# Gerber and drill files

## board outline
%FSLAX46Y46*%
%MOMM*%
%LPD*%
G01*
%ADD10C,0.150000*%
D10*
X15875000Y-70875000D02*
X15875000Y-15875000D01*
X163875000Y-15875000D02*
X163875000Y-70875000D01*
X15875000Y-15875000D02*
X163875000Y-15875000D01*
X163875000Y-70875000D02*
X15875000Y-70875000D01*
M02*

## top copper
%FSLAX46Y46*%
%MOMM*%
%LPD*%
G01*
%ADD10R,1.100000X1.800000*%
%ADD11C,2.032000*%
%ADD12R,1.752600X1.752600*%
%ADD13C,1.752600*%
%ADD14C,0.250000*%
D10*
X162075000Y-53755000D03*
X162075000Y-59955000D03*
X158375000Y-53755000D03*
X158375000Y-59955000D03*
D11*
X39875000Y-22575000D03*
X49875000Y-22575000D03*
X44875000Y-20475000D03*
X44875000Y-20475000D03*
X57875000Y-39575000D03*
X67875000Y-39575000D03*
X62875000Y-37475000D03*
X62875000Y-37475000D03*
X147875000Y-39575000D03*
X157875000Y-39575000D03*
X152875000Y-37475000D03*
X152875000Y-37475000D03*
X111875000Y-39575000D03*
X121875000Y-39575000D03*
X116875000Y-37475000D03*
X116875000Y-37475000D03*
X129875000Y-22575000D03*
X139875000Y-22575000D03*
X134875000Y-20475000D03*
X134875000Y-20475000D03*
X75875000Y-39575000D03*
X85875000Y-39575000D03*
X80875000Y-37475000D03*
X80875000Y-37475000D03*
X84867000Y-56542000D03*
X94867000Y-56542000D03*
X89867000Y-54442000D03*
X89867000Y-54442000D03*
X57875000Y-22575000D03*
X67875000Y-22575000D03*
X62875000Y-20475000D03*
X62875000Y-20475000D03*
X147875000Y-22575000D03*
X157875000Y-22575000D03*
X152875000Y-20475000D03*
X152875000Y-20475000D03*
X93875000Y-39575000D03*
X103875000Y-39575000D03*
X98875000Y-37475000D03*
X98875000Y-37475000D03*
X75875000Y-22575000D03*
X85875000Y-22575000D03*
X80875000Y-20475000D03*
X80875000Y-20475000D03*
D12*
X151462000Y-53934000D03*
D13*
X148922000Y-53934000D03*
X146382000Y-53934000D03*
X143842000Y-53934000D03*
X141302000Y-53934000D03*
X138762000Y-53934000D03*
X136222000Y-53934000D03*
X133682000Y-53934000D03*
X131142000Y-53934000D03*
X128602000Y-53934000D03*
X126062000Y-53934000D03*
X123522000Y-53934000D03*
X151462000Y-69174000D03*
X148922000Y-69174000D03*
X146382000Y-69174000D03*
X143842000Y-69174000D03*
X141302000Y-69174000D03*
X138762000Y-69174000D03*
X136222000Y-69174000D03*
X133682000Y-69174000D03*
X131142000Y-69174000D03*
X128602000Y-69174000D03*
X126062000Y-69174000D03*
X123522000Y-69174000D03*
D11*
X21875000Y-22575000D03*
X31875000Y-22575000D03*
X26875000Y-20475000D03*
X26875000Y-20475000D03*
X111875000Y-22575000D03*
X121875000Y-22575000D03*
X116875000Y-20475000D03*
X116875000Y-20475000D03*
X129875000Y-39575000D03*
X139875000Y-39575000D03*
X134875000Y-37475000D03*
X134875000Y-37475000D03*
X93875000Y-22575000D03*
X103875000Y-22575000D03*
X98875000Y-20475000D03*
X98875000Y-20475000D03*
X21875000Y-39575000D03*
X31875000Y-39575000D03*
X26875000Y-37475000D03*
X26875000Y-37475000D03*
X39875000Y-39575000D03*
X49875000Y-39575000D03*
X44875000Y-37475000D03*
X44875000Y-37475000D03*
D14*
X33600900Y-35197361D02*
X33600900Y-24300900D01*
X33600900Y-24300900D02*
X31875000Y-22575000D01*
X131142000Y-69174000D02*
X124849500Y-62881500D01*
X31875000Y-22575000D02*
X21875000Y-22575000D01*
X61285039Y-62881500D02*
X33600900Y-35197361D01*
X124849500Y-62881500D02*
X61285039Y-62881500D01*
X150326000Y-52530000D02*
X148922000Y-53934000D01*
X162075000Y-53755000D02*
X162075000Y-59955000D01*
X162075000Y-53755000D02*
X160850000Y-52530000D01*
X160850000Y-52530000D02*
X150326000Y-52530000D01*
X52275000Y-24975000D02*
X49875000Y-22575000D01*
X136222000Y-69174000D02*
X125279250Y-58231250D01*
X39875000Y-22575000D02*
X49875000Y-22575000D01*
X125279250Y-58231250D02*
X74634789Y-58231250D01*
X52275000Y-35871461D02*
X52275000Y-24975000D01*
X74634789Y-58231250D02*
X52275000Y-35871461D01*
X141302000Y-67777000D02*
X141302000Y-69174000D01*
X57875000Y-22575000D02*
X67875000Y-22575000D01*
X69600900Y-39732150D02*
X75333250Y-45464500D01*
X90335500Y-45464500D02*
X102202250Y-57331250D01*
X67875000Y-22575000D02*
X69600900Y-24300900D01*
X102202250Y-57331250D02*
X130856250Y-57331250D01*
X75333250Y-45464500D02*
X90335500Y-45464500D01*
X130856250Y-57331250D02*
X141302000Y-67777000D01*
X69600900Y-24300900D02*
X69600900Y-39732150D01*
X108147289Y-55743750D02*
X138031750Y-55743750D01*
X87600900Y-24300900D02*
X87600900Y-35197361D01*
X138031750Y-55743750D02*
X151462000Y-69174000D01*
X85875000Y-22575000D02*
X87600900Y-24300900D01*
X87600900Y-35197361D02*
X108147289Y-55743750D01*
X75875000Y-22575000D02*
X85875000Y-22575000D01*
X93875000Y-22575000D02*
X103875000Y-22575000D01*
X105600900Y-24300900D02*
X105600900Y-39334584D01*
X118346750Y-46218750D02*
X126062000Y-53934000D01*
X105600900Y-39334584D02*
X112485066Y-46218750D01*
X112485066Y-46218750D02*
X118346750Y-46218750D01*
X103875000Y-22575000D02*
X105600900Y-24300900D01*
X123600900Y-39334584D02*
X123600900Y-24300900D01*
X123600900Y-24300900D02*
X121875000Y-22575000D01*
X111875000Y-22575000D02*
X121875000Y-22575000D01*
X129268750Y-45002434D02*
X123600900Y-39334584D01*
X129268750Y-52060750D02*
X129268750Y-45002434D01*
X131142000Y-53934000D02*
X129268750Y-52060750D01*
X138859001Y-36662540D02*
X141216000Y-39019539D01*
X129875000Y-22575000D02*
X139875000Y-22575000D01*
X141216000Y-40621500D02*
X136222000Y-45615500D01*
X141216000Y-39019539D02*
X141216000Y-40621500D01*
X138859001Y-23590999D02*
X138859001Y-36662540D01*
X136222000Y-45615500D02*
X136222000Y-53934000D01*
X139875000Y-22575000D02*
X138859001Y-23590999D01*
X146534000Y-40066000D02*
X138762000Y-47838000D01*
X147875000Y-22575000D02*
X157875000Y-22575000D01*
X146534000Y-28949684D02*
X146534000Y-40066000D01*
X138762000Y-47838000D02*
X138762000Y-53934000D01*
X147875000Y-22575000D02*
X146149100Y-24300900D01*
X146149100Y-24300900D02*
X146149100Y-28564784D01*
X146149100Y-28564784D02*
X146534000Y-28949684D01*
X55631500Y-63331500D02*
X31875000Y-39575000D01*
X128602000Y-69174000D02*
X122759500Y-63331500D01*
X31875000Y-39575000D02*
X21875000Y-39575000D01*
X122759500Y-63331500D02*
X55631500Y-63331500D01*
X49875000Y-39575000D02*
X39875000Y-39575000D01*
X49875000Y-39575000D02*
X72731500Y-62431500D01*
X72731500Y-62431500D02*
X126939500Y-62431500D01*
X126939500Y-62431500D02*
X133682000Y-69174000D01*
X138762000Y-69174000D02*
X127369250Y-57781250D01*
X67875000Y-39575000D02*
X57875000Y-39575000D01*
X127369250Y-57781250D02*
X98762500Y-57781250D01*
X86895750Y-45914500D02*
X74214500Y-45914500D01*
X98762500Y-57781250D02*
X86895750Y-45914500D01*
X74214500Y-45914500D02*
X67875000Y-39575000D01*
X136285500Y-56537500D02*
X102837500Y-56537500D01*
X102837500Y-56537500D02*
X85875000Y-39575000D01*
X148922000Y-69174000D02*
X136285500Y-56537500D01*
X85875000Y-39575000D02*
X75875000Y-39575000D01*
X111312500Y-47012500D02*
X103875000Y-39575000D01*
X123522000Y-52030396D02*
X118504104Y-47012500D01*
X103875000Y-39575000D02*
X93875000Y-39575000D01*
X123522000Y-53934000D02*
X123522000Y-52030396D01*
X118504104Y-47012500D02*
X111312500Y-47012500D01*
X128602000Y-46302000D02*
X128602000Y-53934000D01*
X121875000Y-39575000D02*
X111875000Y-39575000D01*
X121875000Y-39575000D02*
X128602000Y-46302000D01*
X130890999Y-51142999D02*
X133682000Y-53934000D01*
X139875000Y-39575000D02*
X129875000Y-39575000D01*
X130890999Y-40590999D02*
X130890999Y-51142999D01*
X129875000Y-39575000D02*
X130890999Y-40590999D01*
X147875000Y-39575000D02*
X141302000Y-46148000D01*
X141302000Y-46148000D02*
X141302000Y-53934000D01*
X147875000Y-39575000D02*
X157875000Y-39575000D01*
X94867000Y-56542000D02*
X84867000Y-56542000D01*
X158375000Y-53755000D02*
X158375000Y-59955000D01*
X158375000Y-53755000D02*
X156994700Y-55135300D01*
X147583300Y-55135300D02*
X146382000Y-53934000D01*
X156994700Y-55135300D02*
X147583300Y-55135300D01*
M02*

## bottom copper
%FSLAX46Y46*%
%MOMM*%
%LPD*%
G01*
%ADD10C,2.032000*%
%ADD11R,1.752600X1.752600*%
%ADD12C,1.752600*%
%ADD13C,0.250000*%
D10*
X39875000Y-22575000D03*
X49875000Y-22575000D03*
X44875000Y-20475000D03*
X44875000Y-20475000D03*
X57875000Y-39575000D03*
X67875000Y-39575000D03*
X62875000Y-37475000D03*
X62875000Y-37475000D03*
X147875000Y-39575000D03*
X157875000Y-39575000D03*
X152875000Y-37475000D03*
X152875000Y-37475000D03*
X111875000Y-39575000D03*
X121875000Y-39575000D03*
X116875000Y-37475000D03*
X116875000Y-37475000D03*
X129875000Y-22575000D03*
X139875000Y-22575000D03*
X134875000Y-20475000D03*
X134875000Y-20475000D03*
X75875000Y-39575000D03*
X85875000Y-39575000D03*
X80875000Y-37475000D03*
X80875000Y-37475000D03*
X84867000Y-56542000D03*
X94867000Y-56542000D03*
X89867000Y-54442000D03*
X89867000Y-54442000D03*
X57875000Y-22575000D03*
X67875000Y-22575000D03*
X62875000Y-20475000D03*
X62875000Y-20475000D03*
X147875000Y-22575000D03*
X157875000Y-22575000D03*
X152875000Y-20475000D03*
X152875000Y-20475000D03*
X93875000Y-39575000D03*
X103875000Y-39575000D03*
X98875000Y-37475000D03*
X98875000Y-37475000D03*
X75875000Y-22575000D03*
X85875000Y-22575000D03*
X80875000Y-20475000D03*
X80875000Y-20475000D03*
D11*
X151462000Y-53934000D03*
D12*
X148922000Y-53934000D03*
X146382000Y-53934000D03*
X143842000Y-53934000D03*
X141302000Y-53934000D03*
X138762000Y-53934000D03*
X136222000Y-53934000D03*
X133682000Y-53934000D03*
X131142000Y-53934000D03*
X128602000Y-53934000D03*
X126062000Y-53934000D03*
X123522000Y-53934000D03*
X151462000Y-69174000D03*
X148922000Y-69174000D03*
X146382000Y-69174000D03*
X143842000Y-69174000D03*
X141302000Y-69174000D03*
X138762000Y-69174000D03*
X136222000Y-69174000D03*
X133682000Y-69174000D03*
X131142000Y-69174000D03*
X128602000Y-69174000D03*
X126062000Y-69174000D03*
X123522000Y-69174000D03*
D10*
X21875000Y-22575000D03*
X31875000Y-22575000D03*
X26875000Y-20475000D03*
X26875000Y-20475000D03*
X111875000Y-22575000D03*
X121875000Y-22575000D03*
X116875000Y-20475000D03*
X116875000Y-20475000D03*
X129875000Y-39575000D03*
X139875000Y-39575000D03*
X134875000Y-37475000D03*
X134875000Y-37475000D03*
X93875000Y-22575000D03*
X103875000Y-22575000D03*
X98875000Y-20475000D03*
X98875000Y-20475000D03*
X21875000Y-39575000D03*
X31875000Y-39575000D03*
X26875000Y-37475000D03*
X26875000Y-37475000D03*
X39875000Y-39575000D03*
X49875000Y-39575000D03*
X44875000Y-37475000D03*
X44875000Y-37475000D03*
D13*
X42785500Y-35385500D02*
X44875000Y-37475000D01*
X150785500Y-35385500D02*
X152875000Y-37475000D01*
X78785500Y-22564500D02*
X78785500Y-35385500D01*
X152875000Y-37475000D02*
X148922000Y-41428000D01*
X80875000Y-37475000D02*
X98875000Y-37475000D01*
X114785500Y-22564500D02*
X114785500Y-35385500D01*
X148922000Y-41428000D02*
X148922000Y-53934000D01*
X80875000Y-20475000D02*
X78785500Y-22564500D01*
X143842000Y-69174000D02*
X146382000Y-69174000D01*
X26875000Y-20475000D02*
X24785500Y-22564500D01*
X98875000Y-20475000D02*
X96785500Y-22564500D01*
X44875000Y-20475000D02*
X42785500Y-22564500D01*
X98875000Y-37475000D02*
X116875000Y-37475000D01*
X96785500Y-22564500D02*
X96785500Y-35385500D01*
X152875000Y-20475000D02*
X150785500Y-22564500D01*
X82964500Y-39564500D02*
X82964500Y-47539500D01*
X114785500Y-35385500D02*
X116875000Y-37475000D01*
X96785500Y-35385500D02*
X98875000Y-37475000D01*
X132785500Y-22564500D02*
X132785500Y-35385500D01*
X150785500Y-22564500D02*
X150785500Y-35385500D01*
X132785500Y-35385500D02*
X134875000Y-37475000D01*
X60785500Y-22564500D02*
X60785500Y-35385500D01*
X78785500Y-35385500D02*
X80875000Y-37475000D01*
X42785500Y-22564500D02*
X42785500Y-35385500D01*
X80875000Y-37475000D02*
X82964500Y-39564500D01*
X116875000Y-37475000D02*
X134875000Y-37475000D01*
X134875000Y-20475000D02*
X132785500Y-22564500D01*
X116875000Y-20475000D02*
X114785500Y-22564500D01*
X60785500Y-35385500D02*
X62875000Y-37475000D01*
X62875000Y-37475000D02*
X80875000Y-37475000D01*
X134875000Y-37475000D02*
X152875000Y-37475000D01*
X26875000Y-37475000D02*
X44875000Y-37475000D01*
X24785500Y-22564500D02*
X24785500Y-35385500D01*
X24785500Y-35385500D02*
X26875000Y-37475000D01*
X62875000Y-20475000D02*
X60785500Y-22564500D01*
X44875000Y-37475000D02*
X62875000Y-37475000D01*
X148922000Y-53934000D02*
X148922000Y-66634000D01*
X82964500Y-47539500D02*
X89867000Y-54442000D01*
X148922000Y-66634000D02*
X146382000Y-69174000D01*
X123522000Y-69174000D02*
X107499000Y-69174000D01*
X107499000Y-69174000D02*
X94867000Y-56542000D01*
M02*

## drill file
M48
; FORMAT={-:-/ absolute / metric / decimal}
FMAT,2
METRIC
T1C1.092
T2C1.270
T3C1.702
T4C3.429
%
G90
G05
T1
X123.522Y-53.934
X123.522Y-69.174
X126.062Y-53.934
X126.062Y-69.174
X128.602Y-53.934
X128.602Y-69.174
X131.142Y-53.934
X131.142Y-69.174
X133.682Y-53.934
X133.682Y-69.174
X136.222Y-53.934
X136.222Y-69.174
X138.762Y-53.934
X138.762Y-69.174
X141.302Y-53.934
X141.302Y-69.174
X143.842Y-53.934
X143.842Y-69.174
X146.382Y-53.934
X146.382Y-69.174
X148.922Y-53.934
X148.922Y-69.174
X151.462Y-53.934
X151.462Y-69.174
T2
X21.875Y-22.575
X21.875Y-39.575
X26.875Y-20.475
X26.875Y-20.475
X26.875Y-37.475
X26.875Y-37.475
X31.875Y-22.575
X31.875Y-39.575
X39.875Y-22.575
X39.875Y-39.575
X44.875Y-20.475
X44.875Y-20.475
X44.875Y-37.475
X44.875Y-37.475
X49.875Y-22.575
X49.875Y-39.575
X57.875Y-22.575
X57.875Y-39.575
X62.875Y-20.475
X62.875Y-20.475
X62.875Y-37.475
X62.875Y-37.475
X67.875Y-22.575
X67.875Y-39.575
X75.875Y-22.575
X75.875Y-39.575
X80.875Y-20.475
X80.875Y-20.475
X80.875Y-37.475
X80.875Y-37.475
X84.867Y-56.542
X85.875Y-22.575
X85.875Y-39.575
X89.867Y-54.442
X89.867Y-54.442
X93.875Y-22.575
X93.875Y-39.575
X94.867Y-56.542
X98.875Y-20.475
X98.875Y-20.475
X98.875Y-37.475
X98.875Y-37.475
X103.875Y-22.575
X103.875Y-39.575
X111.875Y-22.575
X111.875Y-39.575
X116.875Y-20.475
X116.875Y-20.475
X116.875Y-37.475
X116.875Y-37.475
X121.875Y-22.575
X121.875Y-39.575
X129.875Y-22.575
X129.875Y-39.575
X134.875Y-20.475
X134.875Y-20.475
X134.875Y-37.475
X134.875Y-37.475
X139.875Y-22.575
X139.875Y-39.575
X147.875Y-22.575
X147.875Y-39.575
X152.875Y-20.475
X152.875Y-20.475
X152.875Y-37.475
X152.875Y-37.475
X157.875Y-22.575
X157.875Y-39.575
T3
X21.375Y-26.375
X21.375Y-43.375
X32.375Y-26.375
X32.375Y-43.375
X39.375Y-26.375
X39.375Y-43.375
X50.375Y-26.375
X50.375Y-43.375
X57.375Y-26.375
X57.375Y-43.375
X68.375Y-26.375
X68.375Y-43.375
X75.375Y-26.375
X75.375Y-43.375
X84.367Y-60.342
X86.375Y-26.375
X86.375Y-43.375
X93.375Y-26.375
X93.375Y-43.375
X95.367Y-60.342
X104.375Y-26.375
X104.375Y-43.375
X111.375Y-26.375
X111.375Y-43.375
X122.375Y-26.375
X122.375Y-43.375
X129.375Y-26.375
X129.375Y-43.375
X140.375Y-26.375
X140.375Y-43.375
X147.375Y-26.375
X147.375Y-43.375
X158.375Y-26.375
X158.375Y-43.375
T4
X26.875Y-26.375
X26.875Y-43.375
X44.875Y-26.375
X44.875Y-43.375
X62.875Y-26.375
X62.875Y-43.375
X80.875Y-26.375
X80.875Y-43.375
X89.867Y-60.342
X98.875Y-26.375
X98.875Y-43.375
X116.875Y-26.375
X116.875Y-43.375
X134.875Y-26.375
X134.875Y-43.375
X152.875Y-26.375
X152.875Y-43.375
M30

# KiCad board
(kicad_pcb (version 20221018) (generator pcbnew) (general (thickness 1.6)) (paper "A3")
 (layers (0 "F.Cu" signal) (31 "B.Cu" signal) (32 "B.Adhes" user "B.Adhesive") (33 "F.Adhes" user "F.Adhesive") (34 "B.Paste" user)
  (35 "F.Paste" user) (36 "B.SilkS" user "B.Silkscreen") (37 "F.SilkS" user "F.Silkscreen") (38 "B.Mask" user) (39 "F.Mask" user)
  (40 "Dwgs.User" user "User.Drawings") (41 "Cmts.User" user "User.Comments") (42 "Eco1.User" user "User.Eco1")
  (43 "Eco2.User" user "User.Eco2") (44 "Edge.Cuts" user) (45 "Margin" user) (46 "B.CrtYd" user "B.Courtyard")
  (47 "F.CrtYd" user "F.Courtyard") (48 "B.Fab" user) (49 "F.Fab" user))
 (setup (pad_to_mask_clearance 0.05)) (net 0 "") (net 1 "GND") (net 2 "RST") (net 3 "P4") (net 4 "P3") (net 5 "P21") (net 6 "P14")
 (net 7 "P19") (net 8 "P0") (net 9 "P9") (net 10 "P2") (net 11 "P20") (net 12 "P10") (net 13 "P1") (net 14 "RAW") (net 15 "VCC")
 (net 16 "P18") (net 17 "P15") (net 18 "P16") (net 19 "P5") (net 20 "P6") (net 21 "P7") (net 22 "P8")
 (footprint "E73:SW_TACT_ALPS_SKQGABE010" (layer "F.Cu") (at 160.225 56.855 -90)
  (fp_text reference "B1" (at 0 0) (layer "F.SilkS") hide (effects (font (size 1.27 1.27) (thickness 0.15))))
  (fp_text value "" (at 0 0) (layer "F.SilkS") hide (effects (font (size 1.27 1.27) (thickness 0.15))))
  (pad "1" smd rect (at -3.1 -1.85 270) (size 1.8 1.1) (layers "F.Cu" "F.Paste" "F.Mask") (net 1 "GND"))
  (pad "1" smd rect (at 3.1 -1.85 270) (size 1.8 1.1) (layers "F.Cu" "F.Paste" "F.Mask") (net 1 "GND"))
  (pad "2" smd rect (at -3.1 1.85 270) (size 1.8 1.1) (layers "F.Cu" "F.Paste" "F.Mask") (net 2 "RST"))
  (pad "2" smd rect (at 3.1 1.85 270) (size 1.8 1.1) (layers "F.Cu" "F.Paste" "F.Mask") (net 2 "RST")))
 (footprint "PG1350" (layer "F.Cu") (at 44.875 26.375)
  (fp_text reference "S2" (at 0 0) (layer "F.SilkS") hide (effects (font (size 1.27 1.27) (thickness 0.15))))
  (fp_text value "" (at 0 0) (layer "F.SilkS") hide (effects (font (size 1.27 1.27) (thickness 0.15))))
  (pad "" np_thru_hole circle (at -5.5 0) (size 1.7018 1.7018) (drill 1.7018) (layers "*.Cu" "*.Mask"))
  (pad "" np_thru_hole circle (at 0 0) (size 3.429 3.429) (drill 3.429) (layers "*.Cu" "*.Mask"))
  (pad "" np_thru_hole circle (at 5.5 0) (size 1.7018 1.7018) (drill 1.7018) (layers "*.Cu" "*.Mask"))
  (pad "1" thru_hole circle (at -5 -3.8) (size 2.032 2.032) (drill 1.27) (layers "*.Cu" "*.Mask") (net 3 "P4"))
  (pad "1" thru_hole circle (at 5 -3.8) (size 2.032 2.032) (drill 1.27) (layers "*.Cu" "*.Mask") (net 3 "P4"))
  (pad "2" thru_hole circle (at 0 -5.9) (size 2.032 2.032) (drill 1.27) (layers "*.Cu" "*.Mask") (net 1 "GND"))
  (pad "2" thru_hole circle (at 0 -5.9) (size 2.032 2.032) (drill 1.27) (layers "*.Cu" "*.Mask") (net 1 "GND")))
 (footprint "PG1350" (layer "F.Cu") (at 62.875 43.375)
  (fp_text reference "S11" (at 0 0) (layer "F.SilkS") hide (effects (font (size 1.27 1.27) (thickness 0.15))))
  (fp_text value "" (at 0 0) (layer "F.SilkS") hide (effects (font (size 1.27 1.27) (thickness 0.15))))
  (pad "" np_thru_hole circle (at -5.5 0) (size 1.7018 1.7018) (drill 1.7018) (layers "*.Cu" "*.Mask"))
  (pad "" np_thru_hole circle (at 0 0) (size 3.429 3.429) (drill 3.429) (layers "*.Cu" "*.Mask"))
  (pad "" np_thru_hole circle (at 5.5 0) (size 1.7018 1.7018) (drill 1.7018) (layers "*.Cu" "*.Mask"))
  (pad "1" thru_hole circle (at -5 -3.8) (size 2.032 2.032) (drill 1.27) (layers "*.Cu" "*.Mask") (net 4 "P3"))
  (pad "1" thru_hole circle (at 5 -3.8) (size 2.032 2.032) (drill 1.27) (layers "*.Cu" "*.Mask") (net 4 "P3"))
  (pad "2" thru_hole circle (at 0 -5.9) (size 2.032 2.032) (drill 1.27) (layers "*.Cu" "*.Mask") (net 1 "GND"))
  (pad "2" thru_hole circle (at 0 -5.9) (size 2.032 2.032) (drill 1.27) (layers "*.Cu" "*.Mask") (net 1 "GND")))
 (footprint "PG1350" (layer "F.Cu") (at 152.875 43.375)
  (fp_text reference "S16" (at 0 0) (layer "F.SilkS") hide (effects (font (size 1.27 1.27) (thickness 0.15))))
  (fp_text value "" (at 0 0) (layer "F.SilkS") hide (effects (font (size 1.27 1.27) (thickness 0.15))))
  (pad "" np_thru_hole circle (at -5.5 0) (size 1.7018 1.7018) (drill 1.7018) (layers "*.Cu" "*.Mask"))
  (pad "" np_thru_hole circle (at 0 0) (size 3.429 3.429) (drill 3.429) (layers "*.Cu" "*.Mask"))
  (pad "" np_thru_hole circle (at 5.5 0) (size 1.7018 1.7018) (drill 1.7018) (layers "*.Cu" "*.Mask"))
  (pad "1" thru_hole circle (at -5 -3.8) (size 2.032 2.032) (drill 1.27) (layers "*.Cu" "*.Mask") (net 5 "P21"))
  (pad "1" thru_hole circle (at 5 -3.8) (size 2.032 2.032) (drill 1.27) (layers "*.Cu" "*.Mask") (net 5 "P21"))
  (pad "2" thru_hole circle (at 0 -5.9) (size 2.032 2.032) (drill 1.27) (layers "*.Cu" "*.Mask") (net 1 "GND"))
  (pad "2" thru_hole circle (at 0 -5.9) (size 2.032 2.032) (drill 1.27) (layers "*.Cu" "*.Mask") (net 1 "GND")))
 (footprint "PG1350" (layer "F.Cu") (at 116.875 43.375)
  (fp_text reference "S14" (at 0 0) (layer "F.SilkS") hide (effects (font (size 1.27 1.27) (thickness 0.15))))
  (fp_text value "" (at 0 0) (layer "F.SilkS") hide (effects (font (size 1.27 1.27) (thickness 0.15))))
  (pad "" np_thru_hole circle (at -5.5 0) (size 1.7018 1.7018) (drill 1.7018) (layers "*.Cu" "*.Mask"))
  (pad "" np_thru_hole circle (at 0 0) (size 3.429 3.429) (drill 3.429) (layers "*.Cu" "*.Mask"))
  (pad "" np_thru_hole circle (at 5.5 0) (size 1.7018 1.7018) (drill 1.7018) (layers "*.Cu" "*.Mask"))
  (pad "1" thru_hole circle (at -5 -3.8) (size 2.032 2.032) (drill 1.27) (layers "*.Cu" "*.Mask") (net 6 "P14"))
  (pad "1" thru_hole circle (at 5 -3.8) (size 2.032 2.032) (drill 1.27) (layers "*.Cu" "*.Mask") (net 6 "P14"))
  (pad "2" thru_hole circle (at 0 -5.9) (size 2.032 2.032) (drill 1.27) (layers "*.Cu" "*.Mask") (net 1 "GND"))
  (pad "2" thru_hole circle (at 0 -5.9) (size 2.032 2.032) (drill 1.27) (layers "*.Cu" "*.Mask") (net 1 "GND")))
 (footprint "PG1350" (layer "F.Cu") (at 134.875 26.375)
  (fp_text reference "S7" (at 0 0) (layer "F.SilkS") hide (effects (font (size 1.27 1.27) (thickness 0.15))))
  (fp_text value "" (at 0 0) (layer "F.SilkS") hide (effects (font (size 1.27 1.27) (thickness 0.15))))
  (pad "" np_thru_hole circle (at -5.5 0) (size 1.7018 1.7018) (drill 1.7018) (layers "*.Cu" "*.Mask"))
  (pad "" np_thru_hole circle (at 0 0) (size 3.429 3.429) (drill 3.429) (layers "*.Cu" "*.Mask"))
  (pad "" np_thru_hole circle (at 5.5 0) (size 1.7018 1.7018) (drill 1.7018) (layers "*.Cu" "*.Mask"))
  (pad "1" thru_hole circle (at -5 -3.8) (size 2.032 2.032) (drill 1.27) (layers "*.Cu" "*.Mask") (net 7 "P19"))
  (pad "1" thru_hole circle (at 5 -3.8) (size 2.032 2.032) (drill 1.27) (layers "*.Cu" "*.Mask") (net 7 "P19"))
  (pad "2" thru_hole circle (at 0 -5.9) (size 2.032 2.032) (drill 1.27) (layers "*.Cu" "*.Mask") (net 1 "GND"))
  (pad "2" thru_hole circle (at 0 -5.9) (size 2.032 2.032) (drill 1.27) (layers "*.Cu" "*.Mask") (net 1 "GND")))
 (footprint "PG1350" (layer "F.Cu") (at 80.875 43.375)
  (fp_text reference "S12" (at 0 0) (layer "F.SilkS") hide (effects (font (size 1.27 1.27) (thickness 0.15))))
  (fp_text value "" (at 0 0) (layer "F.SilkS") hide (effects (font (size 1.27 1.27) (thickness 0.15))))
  (pad "" np_thru_hole circle (at -5.5 0) (size 1.7018 1.7018) (drill 1.7018) (layers "*.Cu" "*.Mask"))
  (pad "" np_thru_hole circle (at 0 0) (size 3.429 3.429) (drill 3.429) (layers "*.Cu" "*.Mask"))
  (pad "" np_thru_hole circle (at 5.5 0) (size 1.7018 1.7018) (drill 1.7018) (layers "*.Cu" "*.Mask"))
  (pad "1" thru_hole circle (at -5 -3.8) (size 2.032 2.032) (drill 1.27) (layers "*.Cu" "*.Mask") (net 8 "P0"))
  (pad "1" thru_hole circle (at 5 -3.8) (size 2.032 2.032) (drill 1.27) (layers "*.Cu" "*.Mask") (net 8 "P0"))
  (pad "2" thru_hole circle (at 0 -5.9) (size 2.032 2.032) (drill 1.27) (layers "*.Cu" "*.Mask") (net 1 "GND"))
  (pad "2" thru_hole circle (at 0 -5.9) (size 2.032 2.032) (drill 1.27) (layers "*.Cu" "*.Mask") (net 1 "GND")))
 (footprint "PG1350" (layer "F.Cu") (at 89.867 60.342)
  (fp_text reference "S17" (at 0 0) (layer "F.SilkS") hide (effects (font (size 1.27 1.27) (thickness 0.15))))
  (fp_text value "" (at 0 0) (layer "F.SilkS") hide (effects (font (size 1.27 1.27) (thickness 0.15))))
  (pad "" np_thru_hole circle (at -5.5 0) (size 1.7018 1.7018) (drill 1.7018) (layers "*.Cu" "*.Mask"))
  (pad "" np_thru_hole circle (at 0 0) (size 3.429 3.429) (drill 3.429) (layers "*.Cu" "*.Mask"))
  (pad "" np_thru_hole circle (at 5.5 0) (size 1.7018 1.7018) (drill 1.7018) (layers "*.Cu" "*.Mask"))
  (pad "1" thru_hole circle (at -5 -3.8) (size 2.032 2.032) (drill 1.27) (layers "*.Cu" "*.Mask") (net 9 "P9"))
  (pad "1" thru_hole circle (at 5 -3.8) (size 2.032 2.032) (drill 1.27) (layers "*.Cu" "*.Mask") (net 9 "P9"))
  (pad "2" thru_hole circle (at 0 -5.9) (size 2.032 2.032) (drill 1.27) (layers "*.Cu" "*.Mask") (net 1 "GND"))
  (pad "2" thru_hole circle (at 0 -5.9) (size 2.032 2.032) (drill 1.27) (layers "*.Cu" "*.Mask") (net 1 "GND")))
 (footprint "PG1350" (layer "F.Cu") (at 62.875 26.375)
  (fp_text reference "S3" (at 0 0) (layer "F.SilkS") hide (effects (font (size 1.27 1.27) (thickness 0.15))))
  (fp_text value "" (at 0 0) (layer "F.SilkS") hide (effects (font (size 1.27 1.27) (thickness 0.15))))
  (pad "" np_thru_hole circle (at -5.5 0) (size 1.7018 1.7018) (drill 1.7018) (layers "*.Cu" "*.Mask"))
  (pad "" np_thru_hole circle (at 0 0) (size 3.429 3.429) (drill 3.429) (layers "*.Cu" "*.Mask"))
  (pad "" np_thru_hole circle (at 5.5 0) (size 1.7018 1.7018) (drill 1.7018) (layers "*.Cu" "*.Mask"))
  (pad "1" thru_hole circle (at -5 -3.8) (size 2.032 2.032) (drill 1.27) (layers "*.Cu" "*.Mask") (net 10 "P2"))
  (pad "1" thru_hole circle (at 5 -3.8) (size 2.032 2.032) (drill 1.27) (layers "*.Cu" "*.Mask") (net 10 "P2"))
  (pad "2" thru_hole circle (at 0 -5.9) (size 2.032 2.032) (drill 1.27) (layers "*.Cu" "*.Mask") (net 1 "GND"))
  (pad "2" thru_hole circle (at 0 -5.9) (size 2.032 2.032) (drill 1.27) (layers "*.Cu" "*.Mask") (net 1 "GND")))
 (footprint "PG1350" (layer "F.Cu") (at 152.875 26.375)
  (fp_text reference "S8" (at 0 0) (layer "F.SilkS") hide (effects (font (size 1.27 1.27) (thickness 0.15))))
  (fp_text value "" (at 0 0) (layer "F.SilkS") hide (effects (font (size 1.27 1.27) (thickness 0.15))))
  (pad "" np_thru_hole circle (at -5.5 0) (size 1.7018 1.7018) (drill 1.7018) (layers "*.Cu" "*.Mask"))
  (pad "" np_thru_hole circle (at 0 0) (size 3.429 3.429) (drill 3.429) (layers "*.Cu" "*.Mask"))
  (pad "" np_thru_hole circle (at 5.5 0) (size 1.7018 1.7018) (drill 1.7018) (layers "*.Cu" "*.Mask"))
  (pad "1" thru_hole circle (at -5 -3.8) (size 2.032 2.032) (drill 1.27) (layers "*.Cu" "*.Mask") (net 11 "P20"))
  (pad "1" thru_hole circle (at 5 -3.8) (size 2.032 2.032) (drill 1.27) (layers "*.Cu" "*.Mask") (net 11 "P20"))
  (pad "2" thru_hole circle (at 0 -5.9) (size 2.032 2.032) (drill 1.27) (layers "*.Cu" "*.Mask") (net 1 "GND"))
  (pad "2" thru_hole circle (at 0 -5.9) (size 2.032 2.032) (drill 1.27) (layers "*.Cu" "*.Mask") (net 1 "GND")))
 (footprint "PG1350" (layer "F.Cu") (at 98.875 43.375)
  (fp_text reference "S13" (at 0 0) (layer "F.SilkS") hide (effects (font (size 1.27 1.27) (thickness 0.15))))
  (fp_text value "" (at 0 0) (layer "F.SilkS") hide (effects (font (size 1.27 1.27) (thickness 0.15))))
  (pad "" np_thru_hole circle (at -5.5 0) (size 1.7018 1.7018) (drill 1.7018) (layers "*.Cu" "*.Mask"))
  (pad "" np_thru_hole circle (at 0 0) (size 3.429 3.429) (drill 3.429) (layers "*.Cu" "*.Mask"))
  (pad "" np_thru_hole circle (at 5.5 0) (size 1.7018 1.7018) (drill 1.7018) (layers "*.Cu" "*.Mask"))
  (pad "1" thru_hole circle (at -5 -3.8) (size 2.032 2.032) (drill 1.27) (layers "*.Cu" "*.Mask") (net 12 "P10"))
  (pad "1" thru_hole circle (at 5 -3.8) (size 2.032 2.032) (drill 1.27) (layers "*.Cu" "*.Mask") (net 12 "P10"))
  (pad "2" thru_hole circle (at 0 -5.9) (size 2.032 2.032) (drill 1.27) (layers "*.Cu" "*.Mask") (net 1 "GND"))
  (pad "2" thru_hole circle (at 0 -5.9) (size 2.032 2.032) (drill 1.27) (layers "*.Cu" "*.Mask") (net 1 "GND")))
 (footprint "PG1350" (layer "F.Cu") (at 80.875 26.375)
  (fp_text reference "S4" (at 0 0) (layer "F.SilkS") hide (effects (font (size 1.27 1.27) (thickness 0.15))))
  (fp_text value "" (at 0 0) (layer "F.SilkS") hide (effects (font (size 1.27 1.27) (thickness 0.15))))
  (pad "" np_thru_hole circle (at -5.5 0) (size 1.7018 1.7018) (drill 1.7018) (layers "*.Cu" "*.Mask"))
  (pad "" np_thru_hole circle (at 0 0) (size 3.429 3.429) (drill 3.429) (layers "*.Cu" "*.Mask"))
  (pad "" np_thru_hole circle (at 5.5 0) (size 1.7018 1.7018) (drill 1.7018) (layers "*.Cu" "*.Mask"))
  (pad "1" thru_hole circle (at -5 -3.8) (size 2.032 2.032) (drill 1.27) (layers "*.Cu" "*.Mask") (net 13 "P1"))
  (pad "1" thru_hole circle (at 5 -3.8) (size 2.032 2.032) (drill 1.27) (layers "*.Cu" "*.Mask") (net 13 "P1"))
  (pad "2" thru_hole circle (at 0 -5.9) (size 2.032 2.032) (drill 1.27) (layers "*.Cu" "*.Mask") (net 1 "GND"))
  (pad "2" thru_hole circle (at 0 -5.9) (size 2.032 2.032) (drill 1.27) (layers "*.Cu" "*.Mask") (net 1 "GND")))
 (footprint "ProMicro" (layer "F.Cu") (at 137.492 61.554 180)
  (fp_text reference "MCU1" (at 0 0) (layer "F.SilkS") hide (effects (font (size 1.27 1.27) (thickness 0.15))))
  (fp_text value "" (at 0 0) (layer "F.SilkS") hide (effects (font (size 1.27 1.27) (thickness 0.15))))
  (pad "1" thru_hole rect (at -13.97 7.62 180) (size 1.7526 1.7526) (drill 1.0922) (layers "*.Cu" "*.SilkS" "*.Mask") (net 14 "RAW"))
  (pad "2" thru_hole circle (at -11.43 7.62 180) (size 1.7526 1.7526) (drill 1.0922) (layers "*.Cu" "*.SilkS" "*.Mask") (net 1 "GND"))
  (pad "3" thru_hole circle (at -8.89 7.62 180) (size 1.7526 1.7526) (drill 1.0922) (layers "*.Cu" "*.SilkS" "*.Mask") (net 2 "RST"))
  (pad "4" thru_hole circle (at -6.35 7.62 180) (size 1.7526 1.7526) (drill 1.0922) (layers "*.Cu" "*.SilkS" "*.Mask") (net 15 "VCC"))
  (pad "5" thru_hole circle (at -3.81 7.62 180) (size 1.7526 1.7526) (drill 1.0922) (layers "*.Cu" "*.SilkS" "*.Mask") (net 5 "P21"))
  (pad "6" thru_hole circle (at -1.27 7.62 180) (size 1.7526 1.7526) (drill 1.0922) (layers "*.Cu" "*.SilkS" "*.Mask") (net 11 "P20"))
  (pad "7" thru_hole circle (at 1.27 7.62 180) (size 1.7526 1.7526) (drill 1.0922) (layers "*.Cu" "*.SilkS" "*.Mask") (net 7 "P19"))
  (pad "8" thru_hole circle (at 3.81 7.62 180) (size 1.7526 1.7526) (drill 1.0922) (layers "*.Cu" "*.SilkS" "*.Mask") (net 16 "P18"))
  (pad "9" thru_hole circle (at 6.35 7.62 180) (size 1.7526 1.7526) (drill 1.0922) (layers "*.Cu" "*.SilkS" "*.Mask") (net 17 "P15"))
  (pad "10" thru_hole circle (at 8.89 7.62 180) (size 1.7526 1.7526) (drill 1.0922) (layers "*.Cu" "*.SilkS" "*.Mask") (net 6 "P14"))
  (pad "11" thru_hole circle (at 11.43 7.62 180) (size 1.7526 1.7526) (drill 1.0922) (layers "*.Cu" "*.SilkS" "*.Mask") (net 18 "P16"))
  (pad "12" thru_hole circle (at 13.97 7.62 180) (size 1.7526 1.7526) (drill 1.0922) (layers "*.Cu" "*.SilkS" "*.Mask") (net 12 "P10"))
  (pad "13" thru_hole circle (at -13.97 -7.62 180) (size 1.7526 1.7526) (drill 1.0922) (layers "*.Cu" "*.SilkS" "*.Mask") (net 13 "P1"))
  (pad "14" thru_hole circle (at -11.43 -7.62 180) (size 1.7526 1.7526) (drill 1.0922) (layers "*.Cu" "*.SilkS" "*.Mask") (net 8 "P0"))
  (pad "15" thru_hole circle (at -8.89 -7.62 180) (size 1.7526 1.7526) (drill 1.0922) (layers "*.Cu" "*.SilkS" "*.Mask") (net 1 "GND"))
  (pad "16" thru_hole circle (at -6.35 -7.62 180) (size 1.7526 1.7526) (drill 1.0922) (layers "*.Cu" "*.SilkS" "*.Mask") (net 1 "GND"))
  (pad "17" thru_hole circle (at -3.81 -7.62 180) (size 1.7526 1.7526) (drill 1.0922) (layers "*.Cu" "*.SilkS" "*.Mask") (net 10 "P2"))
  (pad "18" thru_hole circle (at -1.27 -7.62 180) (size 1.7526 1.7526) (drill 1.0922) (layers "*.Cu" "*.SilkS" "*.Mask") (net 4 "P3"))
  (pad "19" thru_hole circle (at 1.27 -7.62 180) (size 1.7526 1.7526) (drill 1.0922) (layers "*.Cu" "*.SilkS" "*.Mask") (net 3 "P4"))
  (pad "20" thru_hole circle (at 3.81 -7.62 180) (size 1.7526 1.7526) (drill 1.0922) (layers "*.Cu" "*.SilkS" "*.Mask") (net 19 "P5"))
  (pad "21" thru_hole circle (at 6.35 -7.62 180) (size 1.7526 1.7526) (drill 1.0922) (layers "*.Cu" "*.SilkS" "*.Mask") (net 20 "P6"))
  (pad "22" thru_hole circle (at 8.89 -7.62 180) (size 1.7526 1.7526) (drill 1.0922) (layers "*.Cu" "*.SilkS" "*.Mask") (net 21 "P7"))
  (pad "23" thru_hole circle (at 11.43 -7.62 180) (size 1.7526 1.7526) (drill 1.0922) (layers "*.Cu" "*.SilkS" "*.Mask") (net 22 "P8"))
  (pad "24" thru_hole circle (at 13.97 -7.62 180) (size 1.7526 1.7526) (drill 1.0922) (layers "*.Cu" "*.SilkS" "*.Mask") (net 9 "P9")))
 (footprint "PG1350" (layer "F.Cu") (at 26.875 26.375)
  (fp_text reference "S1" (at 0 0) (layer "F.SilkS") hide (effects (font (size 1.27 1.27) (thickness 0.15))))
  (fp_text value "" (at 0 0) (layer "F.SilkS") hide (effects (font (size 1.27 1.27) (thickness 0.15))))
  (pad "" np_thru_hole circle (at -5.5 0) (size 1.7018 1.7018) (drill 1.7018) (layers "*.Cu" "*.Mask"))
  (pad "" np_thru_hole circle (at 0 0) (size 3.429 3.429) (drill 3.429) (layers "*.Cu" "*.Mask"))
  (pad "" np_thru_hole circle (at 5.5 0) (size 1.7018 1.7018) (drill 1.7018) (layers "*.Cu" "*.Mask"))
  (pad "1" thru_hole circle (at -5 -3.8) (size 2.032 2.032) (drill 1.27) (layers "*.Cu" "*.Mask") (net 20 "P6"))
  (pad "1" thru_hole circle (at 5 -3.8) (size 2.032 2.032) (drill 1.27) (layers "*.Cu" "*.Mask") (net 20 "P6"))
  (pad "2" thru_hole circle (at 0 -5.9) (size 2.032 2.032) (drill 1.27) (layers "*.Cu" "*.Mask") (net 1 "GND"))
  (pad "2" thru_hole circle (at 0 -5.9) (size 2.032 2.032) (drill 1.27) (layers "*.Cu" "*.Mask") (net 1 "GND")))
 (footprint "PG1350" (layer "F.Cu") (at 116.875 26.375)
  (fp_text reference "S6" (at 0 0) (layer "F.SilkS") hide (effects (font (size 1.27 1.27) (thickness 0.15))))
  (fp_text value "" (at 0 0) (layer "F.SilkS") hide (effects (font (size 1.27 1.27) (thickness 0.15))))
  (pad "" np_thru_hole circle (at -5.5 0) (size 1.7018 1.7018) (drill 1.7018) (layers "*.Cu" "*.Mask"))
  (pad "" np_thru_hole circle (at 0 0) (size 3.429 3.429) (drill 3.429) (layers "*.Cu" "*.Mask"))
  (pad "" np_thru_hole circle (at 5.5 0) (size 1.7018 1.7018) (drill 1.7018) (layers "*.Cu" "*.Mask"))
  (pad "1" thru_hole circle (at -5 -3.8) (size 2.032 2.032) (drill 1.27) (layers "*.Cu" "*.Mask") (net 17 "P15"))
  (pad "1" thru_hole circle (at 5 -3.8) (size 2.032 2.032) (drill 1.27) (layers "*.Cu" "*.Mask") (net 17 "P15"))
  (pad "2" thru_hole circle (at 0 -5.9) (size 2.032 2.032) (drill 1.27) (layers "*.Cu" "*.Mask") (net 1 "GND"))
  (pad "2" thru_hole circle (at 0 -5.9) (size 2.032 2.032) (drill 1.27) (layers "*.Cu" "*.Mask") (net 1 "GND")))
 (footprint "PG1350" (layer "F.Cu") (at 134.875 43.375)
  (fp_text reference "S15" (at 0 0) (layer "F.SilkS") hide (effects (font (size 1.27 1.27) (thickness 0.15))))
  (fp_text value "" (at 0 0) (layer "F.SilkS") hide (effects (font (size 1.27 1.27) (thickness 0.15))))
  (pad "" np_thru_hole circle (at -5.5 0) (size 1.7018 1.7018) (drill 1.7018) (layers "*.Cu" "*.Mask"))
  (pad "" np_thru_hole circle (at 0 0) (size 3.429 3.429) (drill 3.429) (layers "*.Cu" "*.Mask"))
  (pad "" np_thru_hole circle (at 5.5 0) (size 1.7018 1.7018) (drill 1.7018) (layers "*.Cu" "*.Mask"))
  (pad "1" thru_hole circle (at -5 -3.8) (size 2.032 2.032) (drill 1.27) (layers "*.Cu" "*.Mask") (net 16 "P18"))
  (pad "1" thru_hole circle (at 5 -3.8) (size 2.032 2.032) (drill 1.27) (layers "*.Cu" "*.Mask") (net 16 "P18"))
  (pad "2" thru_hole circle (at 0 -5.9) (size 2.032 2.032) (drill 1.27) (layers "*.Cu" "*.Mask") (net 1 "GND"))
  (pad "2" thru_hole circle (at 0 -5.9) (size 2.032 2.032) (drill 1.27) (layers "*.Cu" "*.Mask") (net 1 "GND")))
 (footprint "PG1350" (layer "F.Cu") (at 98.875 26.375)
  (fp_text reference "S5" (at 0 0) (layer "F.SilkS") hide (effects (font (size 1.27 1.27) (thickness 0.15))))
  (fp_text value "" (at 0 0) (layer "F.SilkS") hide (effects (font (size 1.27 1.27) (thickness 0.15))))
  (pad "" np_thru_hole circle (at -5.5 0) (size 1.7018 1.7018) (drill 1.7018) (layers "*.Cu" "*.Mask"))
  (pad "" np_thru_hole circle (at 0 0) (size 3.429 3.429) (drill 3.429) (layers "*.Cu" "*.Mask"))
  (pad "" np_thru_hole circle (at 5.5 0) (size 1.7018 1.7018) (drill 1.7018) (layers "*.Cu" "*.Mask"))
  (pad "1" thru_hole circle (at -5 -3.8) (size 2.032 2.032) (drill 1.27) (layers "*.Cu" "*.Mask") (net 18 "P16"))
  (pad "1" thru_hole circle (at 5 -3.8) (size 2.032 2.032) (drill 1.27) (layers "*.Cu" "*.Mask") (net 18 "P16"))
  (pad "2" thru_hole circle (at 0 -5.9) (size 2.032 2.032) (drill 1.27) (layers "*.Cu" "*.Mask") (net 1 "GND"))
  (pad "2" thru_hole circle (at 0 -5.9) (size 2.032 2.032) (drill 1.27) (layers "*.Cu" "*.Mask") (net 1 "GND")))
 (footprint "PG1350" (layer "F.Cu") (at 26.875 43.375)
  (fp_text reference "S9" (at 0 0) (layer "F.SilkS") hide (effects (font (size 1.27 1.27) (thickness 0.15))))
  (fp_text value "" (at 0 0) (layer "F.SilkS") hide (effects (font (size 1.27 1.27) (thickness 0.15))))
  (pad "" np_thru_hole circle (at -5.5 0) (size 1.7018 1.7018) (drill 1.7018) (layers "*.Cu" "*.Mask"))
  (pad "" np_thru_hole circle (at 0 0) (size 3.429 3.429) (drill 3.429) (layers "*.Cu" "*.Mask"))
  (pad "" np_thru_hole circle (at 5.5 0) (size 1.7018 1.7018) (drill 1.7018) (layers "*.Cu" "*.Mask"))
  (pad "1" thru_hole circle (at -5 -3.8) (size 2.032 2.032) (drill 1.27) (layers "*.Cu" "*.Mask") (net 21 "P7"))
  (pad "1" thru_hole circle (at 5 -3.8) (size 2.032 2.032) (drill 1.27) (layers "*.Cu" "*.Mask") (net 21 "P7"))
  (pad "2" thru_hole circle (at 0 -5.9) (size 2.032 2.032) (drill 1.27) (layers "*.Cu" "*.Mask") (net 1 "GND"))
  (pad "2" thru_hole circle (at 0 -5.9) (size 2.032 2.032) (drill 1.27) (layers "*.Cu" "*.Mask") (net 1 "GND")))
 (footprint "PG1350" (layer "F.Cu") (at 44.875 43.375)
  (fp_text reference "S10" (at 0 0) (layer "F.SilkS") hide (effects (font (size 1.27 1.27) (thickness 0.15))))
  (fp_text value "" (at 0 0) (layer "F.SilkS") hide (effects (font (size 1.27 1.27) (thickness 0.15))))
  (pad "" np_thru_hole circle (at -5.5 0) (size 1.7018 1.7018) (drill 1.7018) (layers "*.Cu" "*.Mask"))
  (pad "" np_thru_hole circle (at 0 0) (size 3.429 3.429) (drill 3.429) (layers "*.Cu" "*.Mask"))
  (pad "" np_thru_hole circle (at 5.5 0) (size 1.7018 1.7018) (drill 1.7018) (layers "*.Cu" "*.Mask"))
  (pad "1" thru_hole circle (at -5 -3.8) (size 2.032 2.032) (drill 1.27) (layers "*.Cu" "*.Mask") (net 19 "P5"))
  (pad "1" thru_hole circle (at 5 -3.8) (size 2.032 2.032) (drill 1.27) (layers "*.Cu" "*.Mask") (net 19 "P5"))
  (pad "2" thru_hole circle (at 0 -5.9) (size 2.032 2.032) (drill 1.27) (layers "*.Cu" "*.Mask") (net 1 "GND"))
  (pad "2" thru_hole circle (at 0 -5.9) (size 2.032 2.032) (drill 1.27) (layers "*.Cu" "*.Mask") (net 1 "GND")))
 (gr_line (start 15.875 70.875) (end 15.875 15.875) (stroke (width 0.15) (type solid)) (layer "Edge.Cuts"))
 (gr_line (start 163.875 15.875) (end 163.875 70.875) (stroke (width 0.15) (type solid)) (layer "Edge.Cuts"))
 (gr_line (start 15.875 15.875) (end 163.875 15.875) (stroke (width 0.15) (type solid)) (layer "Edge.Cuts"))
 (gr_line (start 163.875 70.875) (end 15.875 70.875) (stroke (width 0.15) (type solid)) (layer "Edge.Cuts"))
 (segment (start 33.6009 35.197361) (end 33.6009 24.3009) (width 0.25) (layer "F.Cu") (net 20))
 (segment (start 33.6009 24.3009) (end 31.875 22.575) (width 0.25) (layer "F.Cu") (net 20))
 (segment (start 131.142 69.174) (end 124.8495 62.8815) (width 0.25) (layer "F.Cu") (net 20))
 (segment (start 31.875 22.575) (end 21.875 22.575) (width 0.25) (layer "F.Cu") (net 20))
 (segment (start 61.285039 62.8815) (end 33.6009 35.197361) (width 0.25) (layer "F.Cu") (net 20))
 (segment (start 124.8495 62.8815) (end 61.285039 62.8815) (width 0.25) (layer "F.Cu") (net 20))
 (segment (start 150.326 52.53) (end 148.922 53.934) (width 0.25) (layer "F.Cu") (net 1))
 (segment (start 162.075 53.755) (end 162.075 59.955) (width 0.25) (layer "F.Cu") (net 1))
 (segment (start 162.075 53.755) (end 160.85 52.53) (width 0.25) (layer "F.Cu") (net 1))
 (segment (start 160.85 52.53) (end 150.326 52.53) (width 0.25) (layer "F.Cu") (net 1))
 (segment (start 42.7855 35.3855) (end 44.875 37.475) (width 0.25) (layer "B.Cu") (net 1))
 (segment (start 150.7855 35.3855) (end 152.875 37.475) (width 0.25) (layer "B.Cu") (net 1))
 (segment (start 78.7855 22.5645) (end 78.7855 35.3855) (width 0.25) (layer "B.Cu") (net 1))
 (segment (start 152.875 37.475) (end 148.922 41.428) (width 0.25) (layer "B.Cu") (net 1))
 (segment (start 80.875 37.475) (end 98.875 37.475) (width 0.25) (layer "B.Cu") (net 1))
 (segment (start 114.7855 22.5645) (end 114.7855 35.3855) (width 0.25) (layer "B.Cu") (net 1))
 (segment (start 148.922 41.428) (end 148.922 53.934) (width 0.25) (layer "B.Cu") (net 1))
 (segment (start 80.875 20.475) (end 78.7855 22.5645) (width 0.25) (layer "B.Cu") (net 1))
 (segment (start 143.842 69.174) (end 146.382 69.174) (width 0.25) (layer "B.Cu") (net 1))
 (segment (start 26.875 20.475) (end 24.7855 22.5645) (width 0.25) (layer "B.Cu") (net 1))
 (segment (start 98.875 20.475) (end 96.7855 22.5645) (width 0.25) (layer "B.Cu") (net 1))
 (segment (start 44.875 20.475) (end 42.7855 22.5645) (width 0.25) (layer "B.Cu") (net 1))
 (segment (start 98.875 37.475) (end 116.875 37.475) (width 0.25) (layer "B.Cu") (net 1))
 (segment (start 96.7855 22.5645) (end 96.7855 35.3855) (width 0.25) (layer "B.Cu") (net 1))
 (segment (start 152.875 20.475) (end 150.7855 22.5645) (width 0.25) (layer "B.Cu") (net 1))
 (segment (start 82.9645 39.5645) (end 82.9645 47.5395) (width 0.25) (layer "B.Cu") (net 1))
 (segment (start 114.7855 35.3855) (end 116.875 37.475) (width 0.25) (layer "B.Cu") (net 1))
 (segment (start 96.7855 35.3855) (end 98.875 37.475) (width 0.25) (layer "B.Cu") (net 1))
 (segment (start 132.7855 22.5645) (end 132.7855 35.3855) (width 0.25) (layer "B.Cu") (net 1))
 (segment (start 150.7855 22.5645) (end 150.7855 35.3855) (width 0.25) (layer "B.Cu") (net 1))
 (segment (start 132.7855 35.3855) (end 134.875 37.475) (width 0.25) (layer "B.Cu") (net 1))
 (segment (start 60.7855 22.5645) (end 60.7855 35.3855) (width 0.25) (layer "B.Cu") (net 1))
 (segment (start 78.7855 35.3855) (end 80.875 37.475) (width 0.25) (layer "B.Cu") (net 1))
 (segment (start 42.7855 22.5645) (end 42.7855 35.3855) (width 0.25) (layer "B.Cu") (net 1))
 (segment (start 80.875 37.475) (end 82.9645 39.5645) (width 0.25) (layer "B.Cu") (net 1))
 (segment (start 116.875 37.475) (end 134.875 37.475) (width 0.25) (layer "B.Cu") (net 1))
 (segment (start 134.875 20.475) (end 132.7855 22.5645) (width 0.25) (layer "B.Cu") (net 1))
 (segment (start 116.875 20.475) (end 114.7855 22.5645) (width 0.25) (layer "B.Cu") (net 1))
 (segment (start 60.7855 35.3855) (end 62.875 37.475) (width 0.25) (layer "B.Cu") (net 1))
 (segment (start 62.875 37.475) (end 80.875 37.475) (width 0.25) (layer "B.Cu") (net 1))
 (segment (start 134.875 37.475) (end 152.875 37.475) (width 0.25) (layer "B.Cu") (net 1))
 (segment (start 26.875 37.475) (end 44.875 37.475) (width 0.25) (layer "B.Cu") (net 1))
 (segment (start 24.7855 22.5645) (end 24.7855 35.3855) (width 0.25) (layer "B.Cu") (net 1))
 (segment (start 24.7855 35.3855) (end 26.875 37.475) (width 0.25) (layer "B.Cu") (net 1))
 (segment (start 62.875 20.475) (end 60.7855 22.5645) (width 0.25) (layer "B.Cu") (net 1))
 (segment (start 44.875 37.475) (end 62.875 37.475) (width 0.25) (layer "B.Cu") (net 1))
 (segment (start 148.922 53.934) (end 148.922 66.634) (width 0.25) (layer "B.Cu") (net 1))
 (segment (start 82.9645 47.5395) (end 89.867 54.442) (width 0.25) (layer "B.Cu") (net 1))
 (segment (start 148.922 66.634) (end 146.382 69.174) (width 0.25) (layer "B.Cu") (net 1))
 (segment (start 52.275 24.975) (end 49.875 22.575) (width 0.25) (layer "F.Cu") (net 3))
 (segment (start 136.222 69.174) (end 125.27925 58.23125) (width 0.25) (layer "F.Cu") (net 3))
 (segment (start 39.875 22.575) (end 49.875 22.575) (width 0.25) (layer "F.Cu") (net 3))
 (segment (start 125.27925 58.23125) (end 74.634789 58.23125) (width 0.25) (layer "F.Cu") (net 3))
 (segment (start 52.275 35.871461) (end 52.275 24.975) (width 0.25) (layer "F.Cu") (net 3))
 (segment (start 74.634789 58.23125) (end 52.275 35.871461) (width 0.25) (layer "F.Cu") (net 3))
 (segment (start 141.302 67.777) (end 141.302 69.174) (width 0.25) (layer "F.Cu") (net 10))
 (segment (start 57.875 22.575) (end 67.875 22.575) (width 0.25) (layer "F.Cu") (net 10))
 (segment (start 69.6009 39.73215) (end 75.33325 45.4645) (width 0.25) (layer "F.Cu") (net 10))
 (segment (start 90.3355 45.4645) (end 102.20225 57.33125) (width 0.25) (layer "F.Cu") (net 10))
 (segment (start 67.875 22.575) (end 69.6009 24.3009) (width 0.25) (layer "F.Cu") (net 10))
 (segment (start 102.20225 57.33125) (end 130.85625 57.33125) (width 0.25) (layer "F.Cu") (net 10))
 (segment (start 75.33325 45.4645) (end 90.3355 45.4645) (width 0.25) (layer "F.Cu") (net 10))
 (segment (start 130.85625 57.33125) (end 141.302 67.777) (width 0.25) (layer "F.Cu") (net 10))
 (segment (start 69.6009 24.3009) (end 69.6009 39.73215) (width 0.25) (layer "F.Cu") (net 10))
 (segment (start 108.147289 55.74375) (end 138.03175 55.74375) (width 0.25) (layer "F.Cu") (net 13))
 (segment (start 87.6009 24.3009) (end 87.6009 35.197361) (width 0.25) (layer "F.Cu") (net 13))
 (segment (start 138.03175 55.74375) (end 151.462 69.174) (width 0.25) (layer "F.Cu") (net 13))
 (segment (start 85.875 22.575) (end 87.6009 24.3009) (width 0.25) (layer "F.Cu") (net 13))
 (segment (start 87.6009 35.197361) (end 108.147289 55.74375) (width 0.25) (layer "F.Cu") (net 13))
 (segment (start 75.875 22.575) (end 85.875 22.575) (width 0.25) (layer "F.Cu") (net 13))
 (segment (start 93.875 22.575) (end 103.875 22.575) (width 0.25) (layer "F.Cu") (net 18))
 (segment (start 105.6009 24.3009) (end 105.6009 39.334584) (width 0.25) (layer "F.Cu") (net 18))
 (segment (start 118.34675 46.21875) (end 126.062 53.934) (width 0.25) (layer "F.Cu") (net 18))
 (segment (start 105.6009 39.334584) (end 112.485066 46.21875) (width 0.25) (layer "F.Cu") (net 18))
 (segment (start 112.485066 46.21875) (end 118.34675 46.21875) (width 0.25) (layer "F.Cu") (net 18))
 (segment (start 103.875 22.575) (end 105.6009 24.3009) (width 0.25) (layer "F.Cu") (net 18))
 (segment (start 123.6009 39.334584) (end 123.6009 24.3009) (width 0.25) (layer "F.Cu") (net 17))
 (segment (start 123.6009 24.3009) (end 121.875 22.575) (width 0.25) (layer "F.Cu") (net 17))
 (segment (start 111.875 22.575) (end 121.875 22.575) (width 0.25) (layer "F.Cu") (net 17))
 (segment (start 129.26875 45.002434) (end 123.6009 39.334584) (width 0.25) (layer "F.Cu") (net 17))
 (segment (start 129.26875 52.06075) (end 129.26875 45.002434) (width 0.25) (layer "F.Cu") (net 17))
 (segment (start 131.142 53.934) (end 129.26875 52.06075) (width 0.25) (layer "F.Cu") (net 17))
 (segment (start 138.859001 36.66254) (end 141.216 39.019539) (width 0.25) (layer "F.Cu") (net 7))
 (segment (start 129.875 22.575) (end 139.875 22.575) (width 0.25) (layer "F.Cu") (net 7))
 (segment (start 141.216 40.6215) (end 136.222 45.6155) (width 0.25) (layer "F.Cu") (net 7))
 (segment (start 141.216 39.019539) (end 141.216 40.6215) (width 0.25) (layer "F.Cu") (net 7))
 (segment (start 138.859001 23.590999) (end 138.859001 36.66254) (width 0.25) (layer "F.Cu") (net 7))
 (segment (start 136.222 45.6155) (end 136.222 53.934) (width 0.25) (layer "F.Cu") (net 7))
 (segment (start 139.875 22.575) (end 138.859001 23.590999) (width 0.25) (layer "F.Cu") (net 7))
 (segment (start 146.534 40.066) (end 138.762 47.838) (width 0.25) (layer "F.Cu") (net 11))
 (segment (start 147.875 22.575) (end 157.875 22.575) (width 0.25) (layer "F.Cu") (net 11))
 (segment (start 146.534 28.949684) (end 146.534 40.066) (width 0.25) (layer "F.Cu") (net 11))
 (segment (start 138.762 47.838) (end 138.762 53.934) (width 0.25) (layer "F.Cu") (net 11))
 (segment (start 147.875 22.575) (end 146.1491 24.3009) (width 0.25) (layer "F.Cu") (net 11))
 (segment (start 146.1491 24.3009) (end 146.1491 28.564784) (width 0.25) (layer "F.Cu") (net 11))
 (segment (start 146.1491 28.564784) (end 146.534 28.949684) (width 0.25) (layer "F.Cu") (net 11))
 (segment (start 55.6315 63.3315) (end 31.875 39.575) (width 0.25) (layer "F.Cu") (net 21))
 (segment (start 128.602 69.174) (end 122.7595 63.3315) (width 0.25) (layer "F.Cu") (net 21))
 (segment (start 31.875 39.575) (end 21.875 39.575) (width 0.25) (layer "F.Cu") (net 21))
 (segment (start 122.7595 63.3315) (end 55.6315 63.3315) (width 0.25) (layer "F.Cu") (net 21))
 (segment (start 49.875 39.575) (end 39.875 39.575) (width 0.25) (layer "F.Cu") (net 19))
 (segment (start 49.875 39.575) (end 72.7315 62.4315) (width 0.25) (layer "F.Cu") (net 19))
 (segment (start 72.7315 62.4315) (end 126.9395 62.4315) (width 0.25) (layer "F.Cu") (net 19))
 (segment (start 126.9395 62.4315) (end 133.682 69.174) (width 0.25) (layer "F.Cu") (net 19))
 (segment (start 138.762 69.174) (end 127.36925 57.78125) (width 0.25) (layer "F.Cu") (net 4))
 (segment (start 67.875 39.575) (end 57.875 39.575) (width 0.25) (layer "F.Cu") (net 4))
 (segment (start 127.36925 57.78125) (end 98.7625 57.78125) (width 0.25) (layer "F.Cu") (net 4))
 (segment (start 86.89575 45.9145) (end 74.2145 45.9145) (width 0.25) (layer "F.Cu") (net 4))
 (segment (start 98.7625 57.78125) (end 86.89575 45.9145) (width 0.25) (layer "F.Cu") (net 4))
 (segment (start 74.2145 45.9145) (end 67.875 39.575) (width 0.25) (layer "F.Cu") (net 4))
 (segment (start 136.2855 56.5375) (end 102.8375 56.5375) (width 0.25) (layer "F.Cu") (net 8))
 (segment (start 102.8375 56.5375) (end 85.875 39.575) (width 0.25) (layer "F.Cu") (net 8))
 (segment (start 148.922 69.174) (end 136.2855 56.5375) (width 0.25) (layer "F.Cu") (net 8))
 (segment (start 85.875 39.575) (end 75.875 39.575) (width 0.25) (layer "F.Cu") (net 8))
 (segment (start 111.3125 47.0125) (end 103.875 39.575) (width 0.25) (layer "F.Cu") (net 12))
 (segment (start 123.522 52.030396) (end 118.504104 47.0125) (width 0.25) (layer "F.Cu") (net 12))
 (segment (start 103.875 39.575) (end 93.875 39.575) (width 0.25) (layer "F.Cu") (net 12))
 (segment (start 123.522 53.934) (end 123.522 52.030396) (width 0.25) (layer "F.Cu") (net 12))
 (segment (start 118.504104 47.0125) (end 111.3125 47.0125) (width 0.25) (layer "F.Cu") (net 12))
 (segment (start 128.602 46.302) (end 128.602 53.934) (width 0.25) (layer "F.Cu") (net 6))
 (segment (start 121.875 39.575) (end 111.875 39.575) (width 0.25) (layer "F.Cu") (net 6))
 (segment (start 121.875 39.575) (end 128.602 46.302) (width 0.25) (layer "F.Cu") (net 6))
 (segment (start 130.890999 51.142999) (end 133.682 53.934) (width 0.25) (layer "F.Cu") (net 16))
 (segment (start 139.875 39.575) (end 129.875 39.575) (width 0.25) (layer "F.Cu") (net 16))
 (segment (start 130.890999 40.590999) (end 130.890999 51.142999) (width 0.25) (layer "F.Cu") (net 16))
 (segment (start 129.875 39.575) (end 130.890999 40.590999) (width 0.25) (layer "F.Cu") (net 16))
 (segment (start 147.875 39.575) (end 141.302 46.148) (width 0.25) (layer "F.Cu") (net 5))
 (segment (start 141.302 46.148) (end 141.302 53.934) (width 0.25) (layer "F.Cu") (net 5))
 (segment (start 147.875 39.575) (end 157.875 39.575) (width 0.25) (layer "F.Cu") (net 5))
 (segment (start 94.867 56.542) (end 84.867 56.542) (width 0.25) (layer "F.Cu") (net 9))
 (segment (start 123.522 69.174) (end 107.499 69.174) (width 0.25) (layer "B.Cu") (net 9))
 (segment (start 107.499 69.174) (end 94.867 56.542) (width 0.25) (layer "B.Cu") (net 9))
 (segment (start 158.375 53.755) (end 158.375 59.955) (width 0.25) (layer "F.Cu") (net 2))
 (segment (start 158.375 53.755) (end 156.9947 55.1353) (width 0.25) (layer "F.Cu") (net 2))
 (segment (start 147.5833 55.1353) (end 146.382 53.934) (width 0.25) (layer "F.Cu") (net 2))
 (segment (start 156.9947 55.1353) (end 147.5833 55.1353) (width 0.25) (layer "F.Cu") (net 2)))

